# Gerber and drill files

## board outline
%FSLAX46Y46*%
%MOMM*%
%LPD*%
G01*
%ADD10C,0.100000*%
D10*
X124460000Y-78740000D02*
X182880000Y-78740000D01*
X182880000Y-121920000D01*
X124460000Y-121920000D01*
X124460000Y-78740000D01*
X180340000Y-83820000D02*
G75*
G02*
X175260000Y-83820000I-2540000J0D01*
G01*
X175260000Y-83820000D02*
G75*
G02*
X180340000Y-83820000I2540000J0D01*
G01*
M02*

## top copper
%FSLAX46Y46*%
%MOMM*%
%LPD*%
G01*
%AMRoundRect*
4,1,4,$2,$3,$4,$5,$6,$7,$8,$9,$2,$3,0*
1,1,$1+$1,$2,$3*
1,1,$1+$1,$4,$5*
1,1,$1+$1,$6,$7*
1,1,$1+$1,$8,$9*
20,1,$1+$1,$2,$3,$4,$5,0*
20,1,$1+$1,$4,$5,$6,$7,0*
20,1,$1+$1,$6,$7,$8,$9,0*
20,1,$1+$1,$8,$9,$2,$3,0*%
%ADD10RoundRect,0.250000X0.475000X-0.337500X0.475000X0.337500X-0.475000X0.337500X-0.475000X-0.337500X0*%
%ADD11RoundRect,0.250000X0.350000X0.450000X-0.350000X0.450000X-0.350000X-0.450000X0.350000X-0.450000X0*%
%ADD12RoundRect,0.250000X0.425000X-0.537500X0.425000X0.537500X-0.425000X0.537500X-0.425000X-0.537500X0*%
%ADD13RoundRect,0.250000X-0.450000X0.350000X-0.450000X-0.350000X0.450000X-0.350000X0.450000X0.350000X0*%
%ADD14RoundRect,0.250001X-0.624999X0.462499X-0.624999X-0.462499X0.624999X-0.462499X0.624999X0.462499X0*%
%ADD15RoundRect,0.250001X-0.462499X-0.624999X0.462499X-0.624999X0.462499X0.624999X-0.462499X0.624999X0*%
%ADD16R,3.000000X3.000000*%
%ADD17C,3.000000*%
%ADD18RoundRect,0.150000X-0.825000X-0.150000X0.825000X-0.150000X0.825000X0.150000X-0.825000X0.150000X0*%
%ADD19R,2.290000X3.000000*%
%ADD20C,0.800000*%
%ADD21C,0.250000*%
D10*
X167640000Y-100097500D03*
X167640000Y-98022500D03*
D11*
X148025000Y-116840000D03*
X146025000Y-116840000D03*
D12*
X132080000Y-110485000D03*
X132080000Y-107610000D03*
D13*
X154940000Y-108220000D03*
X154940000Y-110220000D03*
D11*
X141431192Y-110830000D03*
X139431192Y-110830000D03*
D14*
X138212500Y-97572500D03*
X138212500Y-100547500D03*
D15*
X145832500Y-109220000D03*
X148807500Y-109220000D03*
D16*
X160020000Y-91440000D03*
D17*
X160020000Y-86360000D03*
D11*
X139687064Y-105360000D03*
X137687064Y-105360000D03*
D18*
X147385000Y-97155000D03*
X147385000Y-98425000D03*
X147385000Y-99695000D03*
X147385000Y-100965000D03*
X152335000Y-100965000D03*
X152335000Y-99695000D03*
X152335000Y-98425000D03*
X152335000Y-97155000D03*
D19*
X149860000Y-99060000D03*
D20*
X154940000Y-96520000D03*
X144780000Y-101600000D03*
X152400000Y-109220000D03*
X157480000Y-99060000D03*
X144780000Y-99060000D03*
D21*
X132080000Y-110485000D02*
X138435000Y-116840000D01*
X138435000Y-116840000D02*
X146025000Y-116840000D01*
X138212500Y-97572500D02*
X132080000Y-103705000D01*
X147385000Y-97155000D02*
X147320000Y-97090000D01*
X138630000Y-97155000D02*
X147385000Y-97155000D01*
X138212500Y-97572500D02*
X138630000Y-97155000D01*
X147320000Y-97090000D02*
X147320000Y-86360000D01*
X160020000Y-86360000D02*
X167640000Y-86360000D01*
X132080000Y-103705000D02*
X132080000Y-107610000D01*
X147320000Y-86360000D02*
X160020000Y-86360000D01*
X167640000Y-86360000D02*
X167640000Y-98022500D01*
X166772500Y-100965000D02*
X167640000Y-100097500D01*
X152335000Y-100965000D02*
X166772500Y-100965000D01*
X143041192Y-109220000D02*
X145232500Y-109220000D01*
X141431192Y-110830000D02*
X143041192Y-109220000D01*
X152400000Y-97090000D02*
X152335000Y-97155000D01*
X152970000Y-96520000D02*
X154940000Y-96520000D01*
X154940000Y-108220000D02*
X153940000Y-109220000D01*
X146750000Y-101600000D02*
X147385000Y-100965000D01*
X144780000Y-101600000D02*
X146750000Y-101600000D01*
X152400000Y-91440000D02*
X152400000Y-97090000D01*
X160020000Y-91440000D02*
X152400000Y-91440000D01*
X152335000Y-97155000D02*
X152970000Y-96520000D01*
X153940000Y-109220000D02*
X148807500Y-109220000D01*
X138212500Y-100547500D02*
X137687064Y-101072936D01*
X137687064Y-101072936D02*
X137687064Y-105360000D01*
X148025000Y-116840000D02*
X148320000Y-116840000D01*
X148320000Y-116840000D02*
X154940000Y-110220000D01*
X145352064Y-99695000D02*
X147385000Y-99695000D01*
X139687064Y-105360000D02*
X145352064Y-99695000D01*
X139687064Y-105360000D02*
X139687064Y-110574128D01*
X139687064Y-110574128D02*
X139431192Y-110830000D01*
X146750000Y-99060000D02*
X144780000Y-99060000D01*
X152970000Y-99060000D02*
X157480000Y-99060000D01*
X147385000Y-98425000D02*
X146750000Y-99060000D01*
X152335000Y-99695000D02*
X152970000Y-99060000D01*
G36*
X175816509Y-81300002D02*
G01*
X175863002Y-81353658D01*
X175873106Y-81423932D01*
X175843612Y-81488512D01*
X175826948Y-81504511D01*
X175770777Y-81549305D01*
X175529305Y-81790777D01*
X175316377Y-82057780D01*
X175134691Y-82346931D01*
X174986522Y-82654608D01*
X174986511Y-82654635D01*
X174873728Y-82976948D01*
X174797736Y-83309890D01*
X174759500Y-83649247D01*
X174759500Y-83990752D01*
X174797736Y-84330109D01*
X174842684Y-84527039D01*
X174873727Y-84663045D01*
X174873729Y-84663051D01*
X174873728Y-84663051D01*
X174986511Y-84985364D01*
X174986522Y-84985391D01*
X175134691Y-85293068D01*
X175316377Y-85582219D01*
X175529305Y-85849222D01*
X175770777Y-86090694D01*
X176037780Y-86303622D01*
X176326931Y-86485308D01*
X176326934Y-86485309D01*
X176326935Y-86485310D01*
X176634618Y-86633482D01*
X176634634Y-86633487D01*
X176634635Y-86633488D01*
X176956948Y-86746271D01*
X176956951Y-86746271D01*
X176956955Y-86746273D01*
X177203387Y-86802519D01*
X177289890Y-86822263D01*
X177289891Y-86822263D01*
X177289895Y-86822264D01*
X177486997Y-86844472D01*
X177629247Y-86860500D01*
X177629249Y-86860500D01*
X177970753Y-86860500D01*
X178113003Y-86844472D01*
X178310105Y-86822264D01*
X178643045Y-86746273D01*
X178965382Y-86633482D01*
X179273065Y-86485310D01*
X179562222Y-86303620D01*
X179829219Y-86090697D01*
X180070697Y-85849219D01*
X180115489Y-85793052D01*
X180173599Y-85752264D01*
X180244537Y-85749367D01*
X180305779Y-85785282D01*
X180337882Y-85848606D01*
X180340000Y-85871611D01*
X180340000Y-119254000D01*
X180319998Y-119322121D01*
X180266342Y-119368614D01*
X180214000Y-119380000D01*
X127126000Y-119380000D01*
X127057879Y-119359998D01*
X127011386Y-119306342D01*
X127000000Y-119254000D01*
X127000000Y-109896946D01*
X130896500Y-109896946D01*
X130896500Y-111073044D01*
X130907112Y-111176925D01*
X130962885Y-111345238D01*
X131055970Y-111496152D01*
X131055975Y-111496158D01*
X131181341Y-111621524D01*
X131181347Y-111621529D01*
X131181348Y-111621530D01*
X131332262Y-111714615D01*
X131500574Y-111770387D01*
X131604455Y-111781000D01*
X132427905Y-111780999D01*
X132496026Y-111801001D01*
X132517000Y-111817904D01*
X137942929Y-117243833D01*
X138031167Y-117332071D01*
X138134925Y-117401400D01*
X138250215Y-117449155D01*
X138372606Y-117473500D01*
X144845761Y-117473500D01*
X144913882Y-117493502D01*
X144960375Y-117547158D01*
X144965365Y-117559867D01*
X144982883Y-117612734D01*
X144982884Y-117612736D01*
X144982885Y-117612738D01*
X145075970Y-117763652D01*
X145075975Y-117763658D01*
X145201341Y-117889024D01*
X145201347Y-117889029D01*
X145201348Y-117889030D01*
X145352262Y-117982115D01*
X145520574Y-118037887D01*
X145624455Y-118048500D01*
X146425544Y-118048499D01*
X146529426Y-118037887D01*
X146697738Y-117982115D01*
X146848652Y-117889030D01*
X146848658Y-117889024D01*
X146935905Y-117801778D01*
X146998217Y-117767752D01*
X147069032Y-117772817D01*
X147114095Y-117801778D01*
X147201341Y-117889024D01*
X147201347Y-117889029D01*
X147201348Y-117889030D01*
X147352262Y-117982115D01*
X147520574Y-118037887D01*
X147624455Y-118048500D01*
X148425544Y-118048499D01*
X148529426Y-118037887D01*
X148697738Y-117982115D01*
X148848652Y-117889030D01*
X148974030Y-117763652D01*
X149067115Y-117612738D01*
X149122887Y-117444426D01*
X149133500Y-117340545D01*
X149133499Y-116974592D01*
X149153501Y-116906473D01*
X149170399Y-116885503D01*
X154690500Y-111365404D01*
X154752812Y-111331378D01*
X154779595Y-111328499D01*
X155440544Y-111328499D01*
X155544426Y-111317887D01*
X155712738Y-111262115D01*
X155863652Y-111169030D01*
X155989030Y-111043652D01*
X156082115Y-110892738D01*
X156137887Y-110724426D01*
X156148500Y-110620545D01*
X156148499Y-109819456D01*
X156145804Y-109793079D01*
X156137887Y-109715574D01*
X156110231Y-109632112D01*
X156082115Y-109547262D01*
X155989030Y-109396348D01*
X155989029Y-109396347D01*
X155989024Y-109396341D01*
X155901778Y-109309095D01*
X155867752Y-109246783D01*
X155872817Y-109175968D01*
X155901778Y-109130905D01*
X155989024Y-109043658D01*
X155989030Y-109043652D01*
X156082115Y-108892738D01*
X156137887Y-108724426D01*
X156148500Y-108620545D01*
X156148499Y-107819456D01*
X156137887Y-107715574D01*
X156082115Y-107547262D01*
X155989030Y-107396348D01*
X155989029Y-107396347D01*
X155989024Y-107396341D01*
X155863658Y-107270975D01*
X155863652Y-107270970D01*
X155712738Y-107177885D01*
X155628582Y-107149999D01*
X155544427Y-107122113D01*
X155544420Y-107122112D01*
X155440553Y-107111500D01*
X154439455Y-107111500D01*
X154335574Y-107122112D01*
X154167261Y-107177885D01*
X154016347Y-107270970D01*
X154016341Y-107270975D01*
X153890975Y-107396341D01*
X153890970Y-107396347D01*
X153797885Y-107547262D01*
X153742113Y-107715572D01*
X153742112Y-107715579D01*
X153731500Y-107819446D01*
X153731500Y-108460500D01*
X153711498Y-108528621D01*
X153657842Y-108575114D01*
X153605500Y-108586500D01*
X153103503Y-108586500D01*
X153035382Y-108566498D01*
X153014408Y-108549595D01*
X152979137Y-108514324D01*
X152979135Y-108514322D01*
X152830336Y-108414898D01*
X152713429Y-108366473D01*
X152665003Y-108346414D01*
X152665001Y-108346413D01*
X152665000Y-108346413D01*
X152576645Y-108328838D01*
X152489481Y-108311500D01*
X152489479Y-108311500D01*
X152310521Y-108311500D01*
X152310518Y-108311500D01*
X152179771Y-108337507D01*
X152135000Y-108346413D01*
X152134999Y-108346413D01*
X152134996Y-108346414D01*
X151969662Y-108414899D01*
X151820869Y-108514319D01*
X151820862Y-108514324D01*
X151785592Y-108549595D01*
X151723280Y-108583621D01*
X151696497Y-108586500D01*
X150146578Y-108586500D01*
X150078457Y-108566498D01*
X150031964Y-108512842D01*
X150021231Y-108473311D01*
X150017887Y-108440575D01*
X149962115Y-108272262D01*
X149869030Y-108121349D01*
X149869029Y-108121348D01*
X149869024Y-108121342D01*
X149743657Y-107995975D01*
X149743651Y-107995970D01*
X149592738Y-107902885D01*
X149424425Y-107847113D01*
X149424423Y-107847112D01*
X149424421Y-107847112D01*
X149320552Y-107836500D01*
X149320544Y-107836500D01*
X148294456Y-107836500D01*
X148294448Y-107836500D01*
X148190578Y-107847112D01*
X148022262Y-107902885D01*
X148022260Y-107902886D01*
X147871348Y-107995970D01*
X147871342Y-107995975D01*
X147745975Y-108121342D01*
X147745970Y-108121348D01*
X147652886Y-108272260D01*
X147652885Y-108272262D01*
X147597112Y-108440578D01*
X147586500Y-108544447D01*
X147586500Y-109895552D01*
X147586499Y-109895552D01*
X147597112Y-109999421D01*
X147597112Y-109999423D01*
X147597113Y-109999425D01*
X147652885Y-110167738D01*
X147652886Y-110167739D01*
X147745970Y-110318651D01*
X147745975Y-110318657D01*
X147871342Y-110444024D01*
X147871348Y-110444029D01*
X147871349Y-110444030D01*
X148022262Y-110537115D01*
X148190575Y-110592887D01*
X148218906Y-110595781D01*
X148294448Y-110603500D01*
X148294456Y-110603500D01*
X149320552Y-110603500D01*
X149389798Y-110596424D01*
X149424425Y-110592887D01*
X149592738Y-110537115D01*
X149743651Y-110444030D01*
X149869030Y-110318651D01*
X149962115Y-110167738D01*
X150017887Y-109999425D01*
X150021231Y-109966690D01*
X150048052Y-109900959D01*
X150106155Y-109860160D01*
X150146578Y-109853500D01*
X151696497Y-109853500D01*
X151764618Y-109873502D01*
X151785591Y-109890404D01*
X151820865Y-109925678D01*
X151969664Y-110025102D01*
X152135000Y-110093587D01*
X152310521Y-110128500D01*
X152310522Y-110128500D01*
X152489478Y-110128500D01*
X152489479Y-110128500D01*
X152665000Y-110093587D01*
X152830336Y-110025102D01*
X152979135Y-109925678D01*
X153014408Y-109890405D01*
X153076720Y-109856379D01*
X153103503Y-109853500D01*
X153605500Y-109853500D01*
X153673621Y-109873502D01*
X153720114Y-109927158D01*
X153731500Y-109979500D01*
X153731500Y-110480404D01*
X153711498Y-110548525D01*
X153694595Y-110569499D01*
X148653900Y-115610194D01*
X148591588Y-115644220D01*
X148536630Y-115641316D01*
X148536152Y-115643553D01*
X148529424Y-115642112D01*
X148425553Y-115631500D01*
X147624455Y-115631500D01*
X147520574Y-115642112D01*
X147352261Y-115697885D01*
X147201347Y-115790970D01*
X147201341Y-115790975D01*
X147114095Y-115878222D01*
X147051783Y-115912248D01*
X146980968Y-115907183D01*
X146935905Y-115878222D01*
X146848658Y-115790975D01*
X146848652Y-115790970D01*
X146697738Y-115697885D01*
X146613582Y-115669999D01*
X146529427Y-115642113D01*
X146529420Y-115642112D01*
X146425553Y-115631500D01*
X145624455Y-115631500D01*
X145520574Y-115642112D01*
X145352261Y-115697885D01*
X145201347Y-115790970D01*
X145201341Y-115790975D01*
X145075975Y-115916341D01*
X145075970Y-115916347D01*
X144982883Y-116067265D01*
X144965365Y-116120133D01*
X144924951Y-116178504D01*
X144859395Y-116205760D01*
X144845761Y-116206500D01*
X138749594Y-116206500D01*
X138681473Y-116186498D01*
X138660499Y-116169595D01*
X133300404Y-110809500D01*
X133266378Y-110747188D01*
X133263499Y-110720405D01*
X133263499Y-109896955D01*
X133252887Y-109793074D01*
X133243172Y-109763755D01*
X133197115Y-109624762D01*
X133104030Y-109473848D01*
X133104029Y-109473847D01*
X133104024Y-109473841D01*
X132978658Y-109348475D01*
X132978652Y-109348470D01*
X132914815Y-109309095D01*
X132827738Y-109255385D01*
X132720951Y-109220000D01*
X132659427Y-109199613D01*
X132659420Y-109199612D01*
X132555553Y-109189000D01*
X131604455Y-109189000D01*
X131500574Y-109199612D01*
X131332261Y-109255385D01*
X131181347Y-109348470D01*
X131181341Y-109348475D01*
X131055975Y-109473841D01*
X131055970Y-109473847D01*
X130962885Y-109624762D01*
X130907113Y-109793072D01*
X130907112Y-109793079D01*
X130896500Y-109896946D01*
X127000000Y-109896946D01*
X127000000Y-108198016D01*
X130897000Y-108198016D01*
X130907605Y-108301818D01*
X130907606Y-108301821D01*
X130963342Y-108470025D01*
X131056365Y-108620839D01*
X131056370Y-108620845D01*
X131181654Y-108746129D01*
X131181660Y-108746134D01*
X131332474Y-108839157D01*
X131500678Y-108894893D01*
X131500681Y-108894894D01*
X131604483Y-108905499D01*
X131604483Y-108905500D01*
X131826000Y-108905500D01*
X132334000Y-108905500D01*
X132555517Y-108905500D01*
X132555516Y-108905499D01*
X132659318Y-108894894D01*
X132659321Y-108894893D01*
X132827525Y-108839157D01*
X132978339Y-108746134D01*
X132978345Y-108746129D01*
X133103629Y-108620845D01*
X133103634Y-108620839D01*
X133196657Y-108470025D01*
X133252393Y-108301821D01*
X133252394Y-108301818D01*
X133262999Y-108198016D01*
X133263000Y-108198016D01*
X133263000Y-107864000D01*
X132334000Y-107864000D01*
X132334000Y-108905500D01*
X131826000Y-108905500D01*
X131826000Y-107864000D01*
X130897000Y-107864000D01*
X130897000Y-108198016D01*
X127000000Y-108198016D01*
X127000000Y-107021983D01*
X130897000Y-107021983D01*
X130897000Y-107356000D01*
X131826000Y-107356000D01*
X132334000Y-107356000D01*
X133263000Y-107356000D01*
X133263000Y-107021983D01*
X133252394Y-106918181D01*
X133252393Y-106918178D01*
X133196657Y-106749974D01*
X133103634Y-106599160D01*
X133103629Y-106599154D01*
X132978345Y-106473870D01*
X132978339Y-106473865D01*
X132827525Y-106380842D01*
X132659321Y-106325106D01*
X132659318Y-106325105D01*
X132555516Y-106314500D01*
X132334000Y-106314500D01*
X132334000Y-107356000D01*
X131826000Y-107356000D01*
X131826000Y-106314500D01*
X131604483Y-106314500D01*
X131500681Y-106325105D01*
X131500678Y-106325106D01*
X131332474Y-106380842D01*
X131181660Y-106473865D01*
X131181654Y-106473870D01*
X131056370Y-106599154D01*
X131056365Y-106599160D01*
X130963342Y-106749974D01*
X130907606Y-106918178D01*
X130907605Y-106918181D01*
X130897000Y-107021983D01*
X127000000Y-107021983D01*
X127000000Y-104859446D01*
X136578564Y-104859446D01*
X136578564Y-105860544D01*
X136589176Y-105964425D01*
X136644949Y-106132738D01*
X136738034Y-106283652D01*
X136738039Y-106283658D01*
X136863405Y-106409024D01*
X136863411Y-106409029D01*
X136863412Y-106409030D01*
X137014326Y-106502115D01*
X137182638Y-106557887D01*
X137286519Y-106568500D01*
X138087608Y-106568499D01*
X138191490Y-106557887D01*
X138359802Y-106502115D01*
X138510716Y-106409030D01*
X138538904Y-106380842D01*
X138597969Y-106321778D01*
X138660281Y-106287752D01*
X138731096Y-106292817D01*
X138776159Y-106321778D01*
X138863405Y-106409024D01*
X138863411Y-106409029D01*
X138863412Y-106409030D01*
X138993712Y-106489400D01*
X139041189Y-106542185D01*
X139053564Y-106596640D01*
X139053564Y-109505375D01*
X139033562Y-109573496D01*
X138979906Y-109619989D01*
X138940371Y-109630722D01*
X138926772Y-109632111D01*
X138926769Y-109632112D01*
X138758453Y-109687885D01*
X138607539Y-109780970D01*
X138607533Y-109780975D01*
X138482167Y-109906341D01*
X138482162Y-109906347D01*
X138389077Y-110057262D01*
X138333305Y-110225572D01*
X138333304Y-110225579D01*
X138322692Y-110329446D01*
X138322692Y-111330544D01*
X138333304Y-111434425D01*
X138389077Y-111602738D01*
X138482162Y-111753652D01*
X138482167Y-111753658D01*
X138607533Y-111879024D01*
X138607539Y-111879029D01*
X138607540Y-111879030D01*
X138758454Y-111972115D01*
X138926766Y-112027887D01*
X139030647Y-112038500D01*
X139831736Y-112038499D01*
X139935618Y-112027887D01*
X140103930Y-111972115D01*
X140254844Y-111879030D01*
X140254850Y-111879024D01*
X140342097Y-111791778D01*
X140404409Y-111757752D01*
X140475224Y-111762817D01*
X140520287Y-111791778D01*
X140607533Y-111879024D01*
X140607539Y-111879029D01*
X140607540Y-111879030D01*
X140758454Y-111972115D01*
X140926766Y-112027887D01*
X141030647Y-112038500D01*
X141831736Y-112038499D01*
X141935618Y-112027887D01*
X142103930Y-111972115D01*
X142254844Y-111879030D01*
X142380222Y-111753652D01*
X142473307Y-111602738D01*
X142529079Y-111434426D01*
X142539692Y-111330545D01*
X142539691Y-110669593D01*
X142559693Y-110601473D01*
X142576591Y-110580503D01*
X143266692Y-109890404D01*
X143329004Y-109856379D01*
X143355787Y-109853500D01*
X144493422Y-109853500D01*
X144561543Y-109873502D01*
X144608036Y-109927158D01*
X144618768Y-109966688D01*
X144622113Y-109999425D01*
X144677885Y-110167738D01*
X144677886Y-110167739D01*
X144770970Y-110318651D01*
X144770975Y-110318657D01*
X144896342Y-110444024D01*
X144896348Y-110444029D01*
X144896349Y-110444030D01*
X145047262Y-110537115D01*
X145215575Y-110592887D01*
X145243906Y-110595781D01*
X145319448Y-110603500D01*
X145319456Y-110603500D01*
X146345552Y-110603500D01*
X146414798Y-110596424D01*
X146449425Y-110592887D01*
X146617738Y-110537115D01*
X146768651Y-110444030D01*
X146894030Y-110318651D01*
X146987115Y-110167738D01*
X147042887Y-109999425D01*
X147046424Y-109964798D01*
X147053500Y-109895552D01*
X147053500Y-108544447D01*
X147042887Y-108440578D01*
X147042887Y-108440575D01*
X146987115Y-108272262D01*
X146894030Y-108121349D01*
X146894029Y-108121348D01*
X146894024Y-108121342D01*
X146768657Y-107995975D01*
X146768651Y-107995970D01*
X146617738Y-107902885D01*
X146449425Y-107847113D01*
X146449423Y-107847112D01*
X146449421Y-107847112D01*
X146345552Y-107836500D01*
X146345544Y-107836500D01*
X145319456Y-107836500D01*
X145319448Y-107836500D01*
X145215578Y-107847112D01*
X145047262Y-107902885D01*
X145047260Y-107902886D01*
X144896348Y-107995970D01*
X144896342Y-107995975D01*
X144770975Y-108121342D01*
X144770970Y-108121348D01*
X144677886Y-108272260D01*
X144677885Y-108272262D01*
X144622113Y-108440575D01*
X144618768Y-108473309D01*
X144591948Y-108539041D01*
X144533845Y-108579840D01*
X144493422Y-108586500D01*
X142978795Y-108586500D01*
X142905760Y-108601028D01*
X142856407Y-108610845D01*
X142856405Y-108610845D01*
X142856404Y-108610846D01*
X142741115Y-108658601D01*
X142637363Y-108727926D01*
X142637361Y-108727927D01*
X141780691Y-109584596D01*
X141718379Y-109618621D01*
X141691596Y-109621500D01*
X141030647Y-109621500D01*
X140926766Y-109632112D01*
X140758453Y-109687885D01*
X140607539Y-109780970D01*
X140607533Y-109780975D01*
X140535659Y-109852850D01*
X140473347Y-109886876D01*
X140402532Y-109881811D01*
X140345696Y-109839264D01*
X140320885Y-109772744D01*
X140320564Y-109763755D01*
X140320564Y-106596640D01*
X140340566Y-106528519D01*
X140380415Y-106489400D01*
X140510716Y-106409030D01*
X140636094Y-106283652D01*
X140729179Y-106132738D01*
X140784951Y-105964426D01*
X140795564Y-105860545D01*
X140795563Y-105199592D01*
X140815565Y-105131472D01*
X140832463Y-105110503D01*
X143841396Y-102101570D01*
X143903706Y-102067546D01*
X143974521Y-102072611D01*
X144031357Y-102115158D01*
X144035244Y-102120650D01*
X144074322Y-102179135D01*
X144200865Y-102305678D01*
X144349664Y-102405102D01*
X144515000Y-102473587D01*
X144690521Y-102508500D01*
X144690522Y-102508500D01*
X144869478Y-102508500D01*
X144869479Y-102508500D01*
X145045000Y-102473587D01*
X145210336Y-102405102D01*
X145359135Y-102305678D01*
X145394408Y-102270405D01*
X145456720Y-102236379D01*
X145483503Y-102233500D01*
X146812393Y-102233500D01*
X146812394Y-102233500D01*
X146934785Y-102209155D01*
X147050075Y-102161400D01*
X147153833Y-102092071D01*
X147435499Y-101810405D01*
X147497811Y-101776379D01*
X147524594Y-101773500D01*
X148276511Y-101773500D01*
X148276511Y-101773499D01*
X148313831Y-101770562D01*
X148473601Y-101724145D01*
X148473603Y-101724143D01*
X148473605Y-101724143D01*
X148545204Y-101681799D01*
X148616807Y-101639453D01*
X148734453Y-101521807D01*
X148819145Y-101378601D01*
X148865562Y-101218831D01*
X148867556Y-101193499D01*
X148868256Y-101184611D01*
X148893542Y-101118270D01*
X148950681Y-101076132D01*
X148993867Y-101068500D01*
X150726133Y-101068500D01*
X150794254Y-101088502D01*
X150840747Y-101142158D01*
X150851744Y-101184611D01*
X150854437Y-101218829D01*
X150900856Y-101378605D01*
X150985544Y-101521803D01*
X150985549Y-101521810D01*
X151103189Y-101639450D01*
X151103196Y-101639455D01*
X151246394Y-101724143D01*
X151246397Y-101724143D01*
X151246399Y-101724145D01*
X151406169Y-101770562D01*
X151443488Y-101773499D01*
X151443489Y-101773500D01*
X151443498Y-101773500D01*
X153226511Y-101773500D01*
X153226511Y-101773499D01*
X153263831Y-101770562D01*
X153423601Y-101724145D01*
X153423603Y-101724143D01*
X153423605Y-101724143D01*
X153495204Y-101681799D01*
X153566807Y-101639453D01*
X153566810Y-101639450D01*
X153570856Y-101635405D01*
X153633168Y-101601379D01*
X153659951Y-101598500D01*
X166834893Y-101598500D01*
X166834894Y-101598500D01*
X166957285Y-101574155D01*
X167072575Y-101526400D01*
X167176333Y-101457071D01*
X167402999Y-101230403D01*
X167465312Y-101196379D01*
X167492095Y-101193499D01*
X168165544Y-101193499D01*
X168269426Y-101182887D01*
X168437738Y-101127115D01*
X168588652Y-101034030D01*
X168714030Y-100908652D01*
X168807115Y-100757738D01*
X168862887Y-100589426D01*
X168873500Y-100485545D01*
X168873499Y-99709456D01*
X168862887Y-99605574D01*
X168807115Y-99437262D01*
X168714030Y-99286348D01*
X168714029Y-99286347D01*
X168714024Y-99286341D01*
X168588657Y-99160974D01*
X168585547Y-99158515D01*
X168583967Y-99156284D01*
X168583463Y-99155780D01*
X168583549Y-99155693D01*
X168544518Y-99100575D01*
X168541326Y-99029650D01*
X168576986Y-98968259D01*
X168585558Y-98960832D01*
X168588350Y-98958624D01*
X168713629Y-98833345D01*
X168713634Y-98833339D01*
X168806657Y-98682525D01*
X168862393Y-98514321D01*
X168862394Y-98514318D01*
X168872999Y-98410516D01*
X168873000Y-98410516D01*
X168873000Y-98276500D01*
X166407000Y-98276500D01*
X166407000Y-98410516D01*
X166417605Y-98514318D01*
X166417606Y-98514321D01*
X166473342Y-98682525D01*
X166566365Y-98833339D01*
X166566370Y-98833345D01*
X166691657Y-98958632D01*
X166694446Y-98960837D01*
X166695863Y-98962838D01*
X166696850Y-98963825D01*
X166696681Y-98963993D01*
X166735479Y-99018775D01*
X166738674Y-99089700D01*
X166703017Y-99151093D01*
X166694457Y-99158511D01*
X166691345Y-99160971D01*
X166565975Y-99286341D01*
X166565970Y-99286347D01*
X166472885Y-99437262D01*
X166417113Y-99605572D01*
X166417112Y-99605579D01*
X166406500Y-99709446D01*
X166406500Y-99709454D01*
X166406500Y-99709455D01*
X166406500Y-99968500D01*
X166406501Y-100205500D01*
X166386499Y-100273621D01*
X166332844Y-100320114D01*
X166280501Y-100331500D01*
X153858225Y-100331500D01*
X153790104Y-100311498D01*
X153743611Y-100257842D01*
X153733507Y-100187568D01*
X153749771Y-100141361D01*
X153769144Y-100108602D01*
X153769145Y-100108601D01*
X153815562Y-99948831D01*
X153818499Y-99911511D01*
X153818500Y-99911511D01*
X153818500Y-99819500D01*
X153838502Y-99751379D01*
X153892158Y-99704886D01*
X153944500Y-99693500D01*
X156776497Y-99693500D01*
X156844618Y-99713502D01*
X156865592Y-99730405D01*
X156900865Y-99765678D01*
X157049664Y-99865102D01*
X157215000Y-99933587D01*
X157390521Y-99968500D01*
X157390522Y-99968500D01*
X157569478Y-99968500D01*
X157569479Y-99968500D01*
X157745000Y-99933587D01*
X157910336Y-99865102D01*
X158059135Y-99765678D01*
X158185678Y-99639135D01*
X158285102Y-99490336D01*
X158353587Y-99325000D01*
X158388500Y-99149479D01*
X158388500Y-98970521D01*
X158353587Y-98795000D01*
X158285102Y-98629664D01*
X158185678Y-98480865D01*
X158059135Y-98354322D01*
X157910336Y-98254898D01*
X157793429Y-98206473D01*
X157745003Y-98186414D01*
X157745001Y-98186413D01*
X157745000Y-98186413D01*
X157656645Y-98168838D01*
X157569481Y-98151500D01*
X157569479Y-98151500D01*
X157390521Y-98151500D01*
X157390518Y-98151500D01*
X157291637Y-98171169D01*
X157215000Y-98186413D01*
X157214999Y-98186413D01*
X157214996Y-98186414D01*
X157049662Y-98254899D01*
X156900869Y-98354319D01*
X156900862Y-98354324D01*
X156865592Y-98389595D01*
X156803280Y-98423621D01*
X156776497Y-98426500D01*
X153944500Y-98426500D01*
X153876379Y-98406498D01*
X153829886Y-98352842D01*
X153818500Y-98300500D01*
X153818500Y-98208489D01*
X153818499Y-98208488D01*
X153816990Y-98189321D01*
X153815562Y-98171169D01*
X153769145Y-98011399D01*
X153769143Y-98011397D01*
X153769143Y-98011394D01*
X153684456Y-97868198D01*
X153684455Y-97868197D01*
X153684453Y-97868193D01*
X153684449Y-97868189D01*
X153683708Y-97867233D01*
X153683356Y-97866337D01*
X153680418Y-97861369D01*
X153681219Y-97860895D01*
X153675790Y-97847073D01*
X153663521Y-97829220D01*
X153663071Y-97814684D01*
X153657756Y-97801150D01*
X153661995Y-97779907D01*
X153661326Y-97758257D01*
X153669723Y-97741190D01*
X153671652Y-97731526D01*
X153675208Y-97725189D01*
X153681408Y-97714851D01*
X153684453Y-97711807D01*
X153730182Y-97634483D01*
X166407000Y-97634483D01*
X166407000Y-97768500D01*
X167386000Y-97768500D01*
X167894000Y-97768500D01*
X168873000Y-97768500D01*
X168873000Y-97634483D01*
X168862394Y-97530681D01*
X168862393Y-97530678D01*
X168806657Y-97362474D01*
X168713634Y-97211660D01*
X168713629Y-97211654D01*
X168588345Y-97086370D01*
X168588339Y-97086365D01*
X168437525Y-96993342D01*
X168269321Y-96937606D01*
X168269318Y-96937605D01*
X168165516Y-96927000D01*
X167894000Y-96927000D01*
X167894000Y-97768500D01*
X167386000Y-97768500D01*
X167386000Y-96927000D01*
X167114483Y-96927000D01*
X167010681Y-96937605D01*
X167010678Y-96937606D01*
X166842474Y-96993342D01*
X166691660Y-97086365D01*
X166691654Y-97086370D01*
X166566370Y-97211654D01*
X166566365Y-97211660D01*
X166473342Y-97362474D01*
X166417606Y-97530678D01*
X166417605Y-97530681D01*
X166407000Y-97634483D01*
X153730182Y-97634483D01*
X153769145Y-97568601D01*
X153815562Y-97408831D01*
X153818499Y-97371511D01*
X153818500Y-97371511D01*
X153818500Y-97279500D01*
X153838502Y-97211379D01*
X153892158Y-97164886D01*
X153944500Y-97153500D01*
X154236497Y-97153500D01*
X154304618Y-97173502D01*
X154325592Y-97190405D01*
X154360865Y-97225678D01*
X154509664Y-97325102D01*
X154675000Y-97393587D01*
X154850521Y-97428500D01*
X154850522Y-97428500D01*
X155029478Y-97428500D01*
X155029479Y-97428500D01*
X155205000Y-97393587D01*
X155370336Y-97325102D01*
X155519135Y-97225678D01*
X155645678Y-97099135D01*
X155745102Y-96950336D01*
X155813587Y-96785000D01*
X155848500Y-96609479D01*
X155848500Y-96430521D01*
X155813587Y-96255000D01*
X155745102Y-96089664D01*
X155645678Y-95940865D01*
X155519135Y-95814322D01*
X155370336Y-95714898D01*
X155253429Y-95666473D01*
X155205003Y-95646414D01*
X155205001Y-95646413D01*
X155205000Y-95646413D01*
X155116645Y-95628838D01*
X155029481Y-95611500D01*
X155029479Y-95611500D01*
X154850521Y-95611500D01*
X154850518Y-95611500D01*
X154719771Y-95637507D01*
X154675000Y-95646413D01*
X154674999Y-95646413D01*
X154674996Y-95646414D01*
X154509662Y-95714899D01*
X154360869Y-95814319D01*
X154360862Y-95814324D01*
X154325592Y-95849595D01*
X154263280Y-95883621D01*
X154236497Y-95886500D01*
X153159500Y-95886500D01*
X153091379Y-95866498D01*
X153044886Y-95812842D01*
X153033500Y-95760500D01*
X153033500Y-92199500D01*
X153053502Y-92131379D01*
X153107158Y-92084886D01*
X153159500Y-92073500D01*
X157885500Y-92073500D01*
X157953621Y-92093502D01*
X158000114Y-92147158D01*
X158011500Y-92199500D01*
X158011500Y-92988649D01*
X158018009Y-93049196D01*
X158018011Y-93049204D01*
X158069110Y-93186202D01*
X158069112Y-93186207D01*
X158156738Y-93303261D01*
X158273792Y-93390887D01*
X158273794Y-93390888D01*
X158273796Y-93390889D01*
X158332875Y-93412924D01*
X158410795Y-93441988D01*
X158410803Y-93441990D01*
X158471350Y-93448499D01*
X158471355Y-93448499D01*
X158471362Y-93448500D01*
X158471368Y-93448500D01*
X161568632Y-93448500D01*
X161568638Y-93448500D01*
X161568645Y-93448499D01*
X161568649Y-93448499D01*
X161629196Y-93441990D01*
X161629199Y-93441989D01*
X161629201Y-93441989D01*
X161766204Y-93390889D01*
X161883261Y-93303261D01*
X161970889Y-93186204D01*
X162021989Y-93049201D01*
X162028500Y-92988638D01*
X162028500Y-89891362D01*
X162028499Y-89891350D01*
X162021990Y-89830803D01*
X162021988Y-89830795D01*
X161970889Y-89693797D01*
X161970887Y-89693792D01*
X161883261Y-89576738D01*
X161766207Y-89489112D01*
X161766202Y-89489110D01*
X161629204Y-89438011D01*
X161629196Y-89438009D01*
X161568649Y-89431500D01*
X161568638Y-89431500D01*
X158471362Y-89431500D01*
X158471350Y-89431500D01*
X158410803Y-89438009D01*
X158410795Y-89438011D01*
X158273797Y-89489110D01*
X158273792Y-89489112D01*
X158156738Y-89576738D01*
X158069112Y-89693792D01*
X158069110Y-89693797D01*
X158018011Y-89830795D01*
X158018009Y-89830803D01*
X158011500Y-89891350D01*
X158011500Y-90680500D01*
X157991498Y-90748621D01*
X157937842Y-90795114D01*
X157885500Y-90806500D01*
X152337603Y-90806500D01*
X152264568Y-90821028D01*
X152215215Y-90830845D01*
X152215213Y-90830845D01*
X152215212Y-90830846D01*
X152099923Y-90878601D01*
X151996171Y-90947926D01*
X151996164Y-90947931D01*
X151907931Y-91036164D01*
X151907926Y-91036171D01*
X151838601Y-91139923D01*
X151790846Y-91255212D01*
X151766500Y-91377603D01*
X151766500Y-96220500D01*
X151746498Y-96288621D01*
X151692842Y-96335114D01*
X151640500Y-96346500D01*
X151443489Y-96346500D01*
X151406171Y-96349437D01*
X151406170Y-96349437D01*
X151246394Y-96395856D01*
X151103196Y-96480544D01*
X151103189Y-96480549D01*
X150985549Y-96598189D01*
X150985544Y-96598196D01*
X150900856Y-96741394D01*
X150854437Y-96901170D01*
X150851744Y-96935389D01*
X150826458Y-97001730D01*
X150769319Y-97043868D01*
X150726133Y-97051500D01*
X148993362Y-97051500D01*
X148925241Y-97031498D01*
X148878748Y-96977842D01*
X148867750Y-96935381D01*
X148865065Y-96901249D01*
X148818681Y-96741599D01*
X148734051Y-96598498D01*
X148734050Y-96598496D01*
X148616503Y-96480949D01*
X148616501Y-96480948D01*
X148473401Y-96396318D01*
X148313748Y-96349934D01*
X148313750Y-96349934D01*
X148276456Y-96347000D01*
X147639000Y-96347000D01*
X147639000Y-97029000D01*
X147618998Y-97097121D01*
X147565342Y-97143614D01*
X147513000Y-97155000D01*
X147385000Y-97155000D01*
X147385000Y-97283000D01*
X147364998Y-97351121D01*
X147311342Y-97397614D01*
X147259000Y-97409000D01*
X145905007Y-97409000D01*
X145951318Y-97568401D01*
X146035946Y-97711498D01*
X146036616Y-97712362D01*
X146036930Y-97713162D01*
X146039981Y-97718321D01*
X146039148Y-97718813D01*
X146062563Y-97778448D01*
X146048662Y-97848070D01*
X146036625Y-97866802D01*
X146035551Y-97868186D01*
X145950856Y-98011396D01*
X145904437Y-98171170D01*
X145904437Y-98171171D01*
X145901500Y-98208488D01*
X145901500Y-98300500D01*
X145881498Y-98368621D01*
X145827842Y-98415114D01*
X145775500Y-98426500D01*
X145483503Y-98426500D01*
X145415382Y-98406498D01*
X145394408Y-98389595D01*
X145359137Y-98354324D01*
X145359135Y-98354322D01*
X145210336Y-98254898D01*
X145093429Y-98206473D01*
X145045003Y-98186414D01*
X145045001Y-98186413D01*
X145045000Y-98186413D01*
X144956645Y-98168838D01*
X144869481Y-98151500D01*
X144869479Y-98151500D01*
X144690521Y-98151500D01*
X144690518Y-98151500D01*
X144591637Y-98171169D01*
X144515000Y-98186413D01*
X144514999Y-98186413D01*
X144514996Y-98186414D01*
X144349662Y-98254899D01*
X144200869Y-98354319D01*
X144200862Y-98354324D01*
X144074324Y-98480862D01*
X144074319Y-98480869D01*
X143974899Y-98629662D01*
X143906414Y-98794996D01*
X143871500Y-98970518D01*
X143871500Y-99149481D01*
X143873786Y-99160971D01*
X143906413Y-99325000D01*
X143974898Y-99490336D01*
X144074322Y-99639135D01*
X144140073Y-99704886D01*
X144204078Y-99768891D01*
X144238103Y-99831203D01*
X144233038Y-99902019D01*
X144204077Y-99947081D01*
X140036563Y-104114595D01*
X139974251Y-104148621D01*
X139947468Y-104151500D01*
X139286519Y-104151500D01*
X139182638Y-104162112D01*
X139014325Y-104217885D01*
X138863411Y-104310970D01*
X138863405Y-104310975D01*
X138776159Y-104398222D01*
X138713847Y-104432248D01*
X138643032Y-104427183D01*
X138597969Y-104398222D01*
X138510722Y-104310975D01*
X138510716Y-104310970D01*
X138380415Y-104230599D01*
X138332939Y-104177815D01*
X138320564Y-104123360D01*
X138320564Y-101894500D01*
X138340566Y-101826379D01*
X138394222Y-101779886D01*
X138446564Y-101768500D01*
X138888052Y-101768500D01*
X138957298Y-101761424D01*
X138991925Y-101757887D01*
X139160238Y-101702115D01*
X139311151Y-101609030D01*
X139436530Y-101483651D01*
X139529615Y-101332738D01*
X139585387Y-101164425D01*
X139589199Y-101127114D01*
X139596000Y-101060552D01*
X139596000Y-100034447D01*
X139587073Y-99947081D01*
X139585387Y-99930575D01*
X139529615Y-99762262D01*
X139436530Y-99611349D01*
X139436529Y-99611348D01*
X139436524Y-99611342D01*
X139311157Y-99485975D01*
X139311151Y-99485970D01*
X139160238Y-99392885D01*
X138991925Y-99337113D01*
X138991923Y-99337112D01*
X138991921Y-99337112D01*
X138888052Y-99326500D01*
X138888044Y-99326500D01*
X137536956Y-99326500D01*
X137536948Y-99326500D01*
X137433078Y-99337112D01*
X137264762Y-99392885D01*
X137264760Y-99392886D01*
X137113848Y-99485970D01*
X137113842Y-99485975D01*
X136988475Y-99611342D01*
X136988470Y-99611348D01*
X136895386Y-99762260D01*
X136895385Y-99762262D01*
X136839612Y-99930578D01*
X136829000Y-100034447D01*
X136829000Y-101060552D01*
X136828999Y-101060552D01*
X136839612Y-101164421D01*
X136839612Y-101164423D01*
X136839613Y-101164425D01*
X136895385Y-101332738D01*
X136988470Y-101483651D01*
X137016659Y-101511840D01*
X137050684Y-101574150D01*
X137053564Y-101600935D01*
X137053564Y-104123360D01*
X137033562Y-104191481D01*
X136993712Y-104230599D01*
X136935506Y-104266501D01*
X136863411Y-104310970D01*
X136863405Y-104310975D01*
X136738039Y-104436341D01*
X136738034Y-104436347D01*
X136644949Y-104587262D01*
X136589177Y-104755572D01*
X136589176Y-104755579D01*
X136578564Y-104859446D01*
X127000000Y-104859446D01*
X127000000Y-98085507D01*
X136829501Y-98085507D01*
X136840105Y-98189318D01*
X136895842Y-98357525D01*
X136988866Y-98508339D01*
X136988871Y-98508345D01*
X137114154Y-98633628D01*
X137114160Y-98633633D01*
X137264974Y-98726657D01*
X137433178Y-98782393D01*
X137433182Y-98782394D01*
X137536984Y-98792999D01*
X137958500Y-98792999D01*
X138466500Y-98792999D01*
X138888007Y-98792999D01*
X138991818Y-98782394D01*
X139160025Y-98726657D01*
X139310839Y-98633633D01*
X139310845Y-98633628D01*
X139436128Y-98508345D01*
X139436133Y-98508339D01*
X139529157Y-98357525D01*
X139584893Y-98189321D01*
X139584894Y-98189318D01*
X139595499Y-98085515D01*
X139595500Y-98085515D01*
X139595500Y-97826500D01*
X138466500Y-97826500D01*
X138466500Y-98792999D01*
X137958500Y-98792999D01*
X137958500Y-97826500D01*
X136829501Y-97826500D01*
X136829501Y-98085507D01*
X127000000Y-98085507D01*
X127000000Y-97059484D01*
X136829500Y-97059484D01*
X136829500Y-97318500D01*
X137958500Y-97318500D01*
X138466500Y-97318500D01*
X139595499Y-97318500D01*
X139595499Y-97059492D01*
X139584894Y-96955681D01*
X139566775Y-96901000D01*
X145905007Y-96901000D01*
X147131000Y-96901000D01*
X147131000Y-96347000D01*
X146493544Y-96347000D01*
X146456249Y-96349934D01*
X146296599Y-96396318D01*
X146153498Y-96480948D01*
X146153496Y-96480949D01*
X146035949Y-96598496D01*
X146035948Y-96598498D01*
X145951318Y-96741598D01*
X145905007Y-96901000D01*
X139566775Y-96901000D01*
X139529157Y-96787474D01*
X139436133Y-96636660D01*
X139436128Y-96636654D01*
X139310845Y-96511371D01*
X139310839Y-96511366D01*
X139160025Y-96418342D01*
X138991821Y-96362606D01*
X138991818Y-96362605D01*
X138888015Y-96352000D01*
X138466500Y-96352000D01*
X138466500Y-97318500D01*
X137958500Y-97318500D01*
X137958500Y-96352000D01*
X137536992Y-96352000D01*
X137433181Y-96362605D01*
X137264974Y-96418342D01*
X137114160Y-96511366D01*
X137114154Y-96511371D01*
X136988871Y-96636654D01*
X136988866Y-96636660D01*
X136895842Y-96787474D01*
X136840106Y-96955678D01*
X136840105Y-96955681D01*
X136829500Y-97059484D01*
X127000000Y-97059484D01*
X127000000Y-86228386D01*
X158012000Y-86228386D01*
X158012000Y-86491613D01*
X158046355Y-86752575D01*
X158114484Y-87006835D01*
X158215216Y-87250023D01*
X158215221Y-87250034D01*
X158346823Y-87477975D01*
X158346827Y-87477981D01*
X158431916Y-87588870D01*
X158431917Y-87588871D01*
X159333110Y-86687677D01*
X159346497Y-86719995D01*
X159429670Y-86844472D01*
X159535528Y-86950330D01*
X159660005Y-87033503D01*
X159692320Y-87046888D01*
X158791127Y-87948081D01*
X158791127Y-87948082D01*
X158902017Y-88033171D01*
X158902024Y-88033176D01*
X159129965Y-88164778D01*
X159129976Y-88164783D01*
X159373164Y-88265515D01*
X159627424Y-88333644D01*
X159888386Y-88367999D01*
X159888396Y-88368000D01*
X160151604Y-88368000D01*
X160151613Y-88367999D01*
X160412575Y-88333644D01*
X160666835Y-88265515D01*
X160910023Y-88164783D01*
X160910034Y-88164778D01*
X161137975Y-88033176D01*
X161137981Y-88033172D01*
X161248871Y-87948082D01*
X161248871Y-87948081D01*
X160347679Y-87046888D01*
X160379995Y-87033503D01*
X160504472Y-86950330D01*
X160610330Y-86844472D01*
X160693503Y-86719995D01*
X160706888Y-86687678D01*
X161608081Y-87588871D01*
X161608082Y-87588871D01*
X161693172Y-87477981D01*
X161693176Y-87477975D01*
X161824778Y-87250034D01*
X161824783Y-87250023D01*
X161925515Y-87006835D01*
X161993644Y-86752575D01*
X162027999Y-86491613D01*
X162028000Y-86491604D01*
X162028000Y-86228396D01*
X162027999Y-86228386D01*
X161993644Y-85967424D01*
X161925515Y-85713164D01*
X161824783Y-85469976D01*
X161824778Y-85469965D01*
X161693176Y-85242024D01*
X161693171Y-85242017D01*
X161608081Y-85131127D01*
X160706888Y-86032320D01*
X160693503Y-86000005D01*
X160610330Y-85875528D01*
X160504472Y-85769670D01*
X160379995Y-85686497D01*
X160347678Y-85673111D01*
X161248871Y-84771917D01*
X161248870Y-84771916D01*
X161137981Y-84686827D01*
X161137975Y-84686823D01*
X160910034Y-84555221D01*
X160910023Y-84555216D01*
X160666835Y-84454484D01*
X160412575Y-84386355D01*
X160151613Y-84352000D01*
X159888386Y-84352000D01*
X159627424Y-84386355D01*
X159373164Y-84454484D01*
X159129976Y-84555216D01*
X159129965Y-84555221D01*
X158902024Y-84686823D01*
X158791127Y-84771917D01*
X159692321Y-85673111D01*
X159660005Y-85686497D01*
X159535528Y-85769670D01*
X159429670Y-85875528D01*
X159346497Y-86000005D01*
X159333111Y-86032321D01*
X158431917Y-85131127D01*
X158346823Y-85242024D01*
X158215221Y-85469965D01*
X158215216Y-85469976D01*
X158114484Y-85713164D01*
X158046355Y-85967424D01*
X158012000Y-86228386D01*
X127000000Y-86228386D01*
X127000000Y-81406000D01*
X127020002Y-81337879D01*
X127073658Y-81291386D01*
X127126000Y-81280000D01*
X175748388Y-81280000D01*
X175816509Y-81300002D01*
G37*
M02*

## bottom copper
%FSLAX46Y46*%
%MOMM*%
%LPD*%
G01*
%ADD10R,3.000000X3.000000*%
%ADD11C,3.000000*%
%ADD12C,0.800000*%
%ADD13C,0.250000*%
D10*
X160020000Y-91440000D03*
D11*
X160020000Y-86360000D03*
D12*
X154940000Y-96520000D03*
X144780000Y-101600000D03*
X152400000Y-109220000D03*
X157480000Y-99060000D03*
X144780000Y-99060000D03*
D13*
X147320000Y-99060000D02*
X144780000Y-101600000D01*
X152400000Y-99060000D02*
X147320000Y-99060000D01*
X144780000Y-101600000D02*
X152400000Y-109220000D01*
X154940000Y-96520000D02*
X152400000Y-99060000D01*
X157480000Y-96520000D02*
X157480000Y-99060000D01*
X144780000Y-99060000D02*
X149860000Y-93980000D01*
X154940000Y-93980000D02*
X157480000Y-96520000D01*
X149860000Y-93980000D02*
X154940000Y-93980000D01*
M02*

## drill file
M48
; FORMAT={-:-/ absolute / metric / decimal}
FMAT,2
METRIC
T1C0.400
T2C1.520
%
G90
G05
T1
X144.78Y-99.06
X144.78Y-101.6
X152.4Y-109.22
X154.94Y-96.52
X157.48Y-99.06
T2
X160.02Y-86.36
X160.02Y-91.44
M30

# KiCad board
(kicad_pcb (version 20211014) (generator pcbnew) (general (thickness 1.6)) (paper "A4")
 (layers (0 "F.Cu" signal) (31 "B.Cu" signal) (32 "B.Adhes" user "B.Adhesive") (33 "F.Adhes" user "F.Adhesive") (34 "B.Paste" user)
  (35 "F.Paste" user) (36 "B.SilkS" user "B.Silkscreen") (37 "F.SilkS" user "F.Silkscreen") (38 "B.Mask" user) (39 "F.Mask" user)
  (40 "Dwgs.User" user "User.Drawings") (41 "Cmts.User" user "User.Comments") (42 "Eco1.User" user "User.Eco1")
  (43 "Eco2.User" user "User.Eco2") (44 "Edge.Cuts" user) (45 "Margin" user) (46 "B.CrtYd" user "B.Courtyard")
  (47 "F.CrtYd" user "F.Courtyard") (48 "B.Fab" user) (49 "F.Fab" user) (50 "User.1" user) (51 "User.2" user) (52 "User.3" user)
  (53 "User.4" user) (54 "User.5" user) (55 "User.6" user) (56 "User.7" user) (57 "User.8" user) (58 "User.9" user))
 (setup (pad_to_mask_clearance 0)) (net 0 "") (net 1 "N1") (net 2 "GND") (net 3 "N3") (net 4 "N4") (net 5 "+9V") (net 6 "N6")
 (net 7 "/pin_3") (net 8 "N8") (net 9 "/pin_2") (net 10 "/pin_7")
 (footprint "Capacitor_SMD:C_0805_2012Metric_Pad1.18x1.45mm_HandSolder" (layer "F.Cu") (at 167.64 99.06 90)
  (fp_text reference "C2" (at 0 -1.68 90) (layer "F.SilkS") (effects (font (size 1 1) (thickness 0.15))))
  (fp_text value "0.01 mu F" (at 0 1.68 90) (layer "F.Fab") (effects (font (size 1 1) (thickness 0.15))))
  (pad "1" smd roundrect (at -1.0375 0 90) (size 1.175 1.45) (layers "F.Cu" "F.Paste" "F.Mask") (roundrect_rratio 0.2127659574) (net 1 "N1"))
  (pad "2" smd roundrect (at 1.0375 0 90) (size 1.175 1.45) (layers "F.Cu" "F.Paste" "F.Mask") (roundrect_rratio 0.2127659574) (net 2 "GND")))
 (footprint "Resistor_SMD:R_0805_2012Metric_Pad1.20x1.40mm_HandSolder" (layer "F.Cu") (at 147.025 116.84 180)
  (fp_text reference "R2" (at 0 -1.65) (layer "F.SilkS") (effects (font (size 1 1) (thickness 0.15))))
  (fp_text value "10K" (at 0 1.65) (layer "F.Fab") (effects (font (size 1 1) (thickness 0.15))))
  (pad "1" smd roundrect (at -1 0 180) (size 1.2 1.4) (layers "F.Cu" "F.Paste" "F.Mask") (roundrect_rratio 0.2083333333) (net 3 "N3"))
  (pad "2" smd roundrect (at 1 0 180) (size 1.2 1.4) (layers "F.Cu" "F.Paste" "F.Mask") (roundrect_rratio 0.2083333333) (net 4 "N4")))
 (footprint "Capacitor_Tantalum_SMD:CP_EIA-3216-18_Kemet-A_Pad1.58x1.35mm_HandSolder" (layer "F.Cu") (at 132.08 109.0475 90)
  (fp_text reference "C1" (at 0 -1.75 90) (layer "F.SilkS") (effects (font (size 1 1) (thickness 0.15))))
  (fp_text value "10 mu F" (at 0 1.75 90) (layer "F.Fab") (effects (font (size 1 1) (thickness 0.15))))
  (pad "1" smd roundrect (at -1.4375 0 90) (size 1.575 1.35) (layers "F.Cu" "F.Paste" "F.Mask") (roundrect_rratio 0.1851851852) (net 4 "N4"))
  (pad "2" smd roundrect (at 1.4375 0 90) (size 1.575 1.35) (layers "F.Cu" "F.Paste" "F.Mask") (roundrect_rratio 0.1851851852) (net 2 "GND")))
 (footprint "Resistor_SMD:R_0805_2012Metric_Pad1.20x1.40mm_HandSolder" (layer "F.Cu") (at 154.94 109.22 -90)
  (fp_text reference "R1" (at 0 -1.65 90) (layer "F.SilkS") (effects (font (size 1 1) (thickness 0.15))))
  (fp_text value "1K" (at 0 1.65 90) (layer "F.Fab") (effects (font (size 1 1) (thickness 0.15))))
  (pad "1" smd roundrect (at -1 0 270) (size 1.2 1.4) (layers "F.Cu" "F.Paste" "F.Mask") (roundrect_rratio 0.2083333333) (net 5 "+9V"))
  (pad "2" smd roundrect (at 1 0 270) (size 1.2 1.4) (layers "F.Cu" "F.Paste" "F.Mask") (roundrect_rratio 0.2083333333) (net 3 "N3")))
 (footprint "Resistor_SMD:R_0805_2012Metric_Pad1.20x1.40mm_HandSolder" (layer "F.Cu") (at 140.431192 110.83 180)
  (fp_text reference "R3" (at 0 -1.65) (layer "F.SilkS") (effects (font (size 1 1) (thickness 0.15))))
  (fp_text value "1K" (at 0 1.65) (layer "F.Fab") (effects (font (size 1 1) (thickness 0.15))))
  (pad "1" smd roundrect (at -1 0 180) (size 1.2 1.4) (layers "F.Cu" "F.Paste" "F.Mask") (roundrect_rratio 0.2083333333) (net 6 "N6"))
  (pad "2" smd roundrect (at 1 0 180) (size 1.2 1.4) (layers "F.Cu" "F.Paste" "F.Mask") (roundrect_rratio 0.2083333333) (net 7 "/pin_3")))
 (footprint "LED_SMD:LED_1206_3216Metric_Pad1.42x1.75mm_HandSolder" (layer "F.Cu") (at 138.2125 99.06 -90)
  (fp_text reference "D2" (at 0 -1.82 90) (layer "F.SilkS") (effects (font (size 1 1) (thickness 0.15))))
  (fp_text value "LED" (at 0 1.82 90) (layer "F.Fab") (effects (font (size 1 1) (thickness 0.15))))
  (pad "1" smd roundrect (at -1.4875 0 270) (size 1.425 1.75) (layers "F.Cu" "F.Paste" "F.Mask") (roundrect_rratio 0.1754392982)
   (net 2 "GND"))
  (pad "2" smd roundrect (at 1.4875 0 270) (size 1.425 1.75) (layers "F.Cu" "F.Paste" "F.Mask") (roundrect_rratio 0.1754392982) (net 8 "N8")))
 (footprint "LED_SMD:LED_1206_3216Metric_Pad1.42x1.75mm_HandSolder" (layer "F.Cu") (at 147.32 109.22)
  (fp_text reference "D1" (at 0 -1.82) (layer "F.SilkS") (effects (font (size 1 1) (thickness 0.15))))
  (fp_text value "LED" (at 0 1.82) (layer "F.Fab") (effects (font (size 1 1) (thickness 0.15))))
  (pad "1" smd roundrect (at -1.4875 0) (size 1.425 1.75) (layers "F.Cu" "F.Paste" "F.Mask") (roundrect_rratio 0.1754392982) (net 6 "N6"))
  (pad "2" smd roundrect (at 1.4875 0) (size 1.425 1.75) (layers "F.Cu" "F.Paste" "F.Mask") (roundrect_rratio 0.1754392982) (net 5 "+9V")))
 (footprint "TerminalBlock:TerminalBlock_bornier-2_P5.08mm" (layer "F.Cu") (at 160.02 91.44 90)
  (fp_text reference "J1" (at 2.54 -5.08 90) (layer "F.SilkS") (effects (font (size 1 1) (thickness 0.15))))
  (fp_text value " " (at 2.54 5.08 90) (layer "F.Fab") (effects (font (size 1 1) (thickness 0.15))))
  (pad "1" thru_hole rect (at 0 0 90) (size 3 3) (drill 1.52) (layers *.Cu *.Mask) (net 5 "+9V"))
  (pad "2" thru_hole circle (at 5.08 0 90) (size 3 3) (drill 1.52) (layers *.Cu *.Mask) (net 2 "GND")))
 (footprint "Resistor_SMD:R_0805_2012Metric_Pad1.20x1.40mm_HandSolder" (layer "F.Cu") (at 138.687064 105.36 180)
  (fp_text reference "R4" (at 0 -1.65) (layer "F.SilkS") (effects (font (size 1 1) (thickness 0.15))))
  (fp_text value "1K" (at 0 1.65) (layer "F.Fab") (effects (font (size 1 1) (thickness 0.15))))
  (pad "1" smd roundrect (at -1 0 180) (size 1.2 1.4) (layers "F.Cu" "F.Paste" "F.Mask") (roundrect_rratio 0.2083333333) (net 7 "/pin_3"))
  (pad "2" smd roundrect (at 1 0 180) (size 1.2 1.4) (layers "F.Cu" "F.Paste" "F.Mask") (roundrect_rratio 0.2083333333) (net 8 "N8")))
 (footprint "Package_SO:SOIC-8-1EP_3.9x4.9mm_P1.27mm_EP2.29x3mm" (layer "F.Cu") (at 149.86 99.06)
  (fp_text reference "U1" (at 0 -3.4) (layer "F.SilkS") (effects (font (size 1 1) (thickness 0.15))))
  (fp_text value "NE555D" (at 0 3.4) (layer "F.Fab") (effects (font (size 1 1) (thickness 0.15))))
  (pad "" smd roundrect (at -0.57 0.75) (size 0.92 1.21) (layers "F.Paste") (roundrect_rratio 0.25))
  (pad "" smd roundrect (at 0.57 -0.75) (size 0.92 1.21) (layers "F.Paste") (roundrect_rratio 0.25))
  (pad "" smd roundrect (at 0.57 0.75) (size 0.92 1.21) (layers "F.Paste") (roundrect_rratio 0.25))
  (pad "" smd roundrect (at -0.57 -0.75) (size 0.92 1.21) (layers "F.Paste") (roundrect_rratio 0.25))
  (pad "1" smd roundrect (at -2.475 -1.905) (size 1.95 0.6) (layers "F.Cu" "F.Paste" "F.Mask") (roundrect_rratio 0.25) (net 2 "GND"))
  (pad "2" smd roundrect (at -2.475 -0.635) (size 1.95 0.6) (layers "F.Cu" "F.Paste" "F.Mask") (roundrect_rratio 0.25) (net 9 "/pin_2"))
  (pad "3" smd roundrect (at -2.475 0.635) (size 1.95 0.6) (layers "F.Cu" "F.Paste" "F.Mask") (roundrect_rratio 0.25) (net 7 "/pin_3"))
  (pad "4" smd roundrect (at -2.475 1.905) (size 1.95 0.6) (layers "F.Cu" "F.Paste" "F.Mask") (roundrect_rratio 0.25) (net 5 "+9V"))
  (pad "5" smd roundrect (at 2.475 1.905) (size 1.95 0.6) (layers "F.Cu" "F.Paste" "F.Mask") (roundrect_rratio 0.25) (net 1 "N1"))
  (pad "6" smd roundrect (at 2.475 0.635) (size 1.95 0.6) (layers "F.Cu" "F.Paste" "F.Mask") (roundrect_rratio 0.25) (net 9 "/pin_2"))
  (pad "7" smd roundrect (at 2.475 -0.635) (size 1.95 0.6) (layers "F.Cu" "F.Paste" "F.Mask") (roundrect_rratio 0.25) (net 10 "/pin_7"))
  (pad "8" smd roundrect (at 2.475 -1.905) (size 1.95 0.6) (layers "F.Cu" "F.Paste" "F.Mask") (roundrect_rratio 0.25) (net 5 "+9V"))
  (pad "9" smd rect (at 0 0) (size 2.29 3) (layers "F.Cu" "F.Mask")))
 (gr_rect (start 124.46 78.74) (end 182.88 121.92) (layer "Edge.Cuts") (width 0.1) (fill none))
 (gr_circle (center 177.8 83.82) (end 180.34 83.82) (layer "Edge.Cuts") (width 0.1) (fill none))
 (segment (start 132.08 110.485) (end 138.435 116.84) (width 0.25) (layer "F.Cu") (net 4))
 (segment (start 138.435 116.84) (end 146.025 116.84) (width 0.25) (layer "F.Cu") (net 4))
 (segment (start 138.2125 97.5725) (end 132.08 103.705) (width 0.25) (layer "F.Cu") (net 2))
 (segment (start 147.385 97.155) (end 147.32 97.09) (width 0.25) (layer "F.Cu") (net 2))
 (segment (start 138.63 97.155) (end 147.385 97.155) (width 0.25) (layer "F.Cu") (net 2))
 (segment (start 138.2125 97.5725) (end 138.63 97.155) (width 0.25) (layer "F.Cu") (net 2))
 (segment (start 147.32 97.09) (end 147.32 86.36) (width 0.25) (layer "F.Cu") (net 2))
 (segment (start 160.02 86.36) (end 167.64 86.36) (width 0.25) (layer "F.Cu") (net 2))
 (segment (start 132.08 103.705) (end 132.08 107.61) (width 0.25) (layer "F.Cu") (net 2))
 (segment (start 147.32 86.36) (end 160.02 86.36) (width 0.25) (layer "F.Cu") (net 2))
 (segment (start 167.64 86.36) (end 167.64 98.0225) (width 0.25) (layer "F.Cu") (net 2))
 (segment (start 166.7725 100.965) (end 167.64 100.0975) (width 0.25) (layer "F.Cu") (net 1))
 (segment (start 152.335 100.965) (end 166.7725 100.965) (width 0.25) (layer "F.Cu") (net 1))
 (segment (start 143.041192 109.22) (end 145.2325 109.22) (width 0.25) (layer "F.Cu") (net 6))
 (segment (start 141.431192 110.83) (end 143.041192 109.22) (width 0.25) (layer "F.Cu") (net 6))
 (segment (start 152.4 97.09) (end 152.335 97.155) (width 0.25) (layer "F.Cu") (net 5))
 (segment (start 152.97 96.52) (end 154.94 96.52) (width 0.25) (layer "F.Cu") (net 5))
 (segment (start 154.94 108.22) (end 153.94 109.22) (width 0.25) (layer "F.Cu") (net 5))
 (segment (start 146.75 101.6) (end 147.385 100.965) (width 0.25) (layer "F.Cu") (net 5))
 (segment (start 144.78 101.6) (end 146.75 101.6) (width 0.25) (layer "F.Cu") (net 5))
 (segment (start 152.4 91.44) (end 152.4 97.09) (width 0.25) (layer "F.Cu") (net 5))
 (segment (start 160.02 91.44) (end 152.4 91.44) (width 0.25) (layer "F.Cu") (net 5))
 (segment (start 152.335 97.155) (end 152.97 96.52) (width 0.25) (layer "F.Cu") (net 5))
 (segment (start 153.94 109.22) (end 148.8075 109.22) (width 0.25) (layer "F.Cu") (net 5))
 (via (at 154.94 96.52) (size 0.8) (drill 0.4) (layers "F.Cu" "B.Cu") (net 5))
 (via (at 144.78 101.6) (size 0.8) (drill 0.4) (layers "F.Cu" "B.Cu") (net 5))
 (via (at 152.4 109.22) (size 0.8) (drill 0.4) (layers "F.Cu" "B.Cu") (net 5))
 (segment (start 147.32 99.06) (end 144.78 101.6) (width 0.25) (layer "B.Cu") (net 5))
 (segment (start 152.4 99.06) (end 147.32 99.06) (width 0.25) (layer "B.Cu") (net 5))
 (segment (start 144.78 101.6) (end 152.4 109.22) (width 0.25) (layer "B.Cu") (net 5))
 (segment (start 154.94 96.52) (end 152.4 99.06) (width 0.25) (layer "B.Cu") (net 5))
 (segment (start 138.2125 100.5475) (end 137.687064 101.072936) (width 0.25) (layer "F.Cu") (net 8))
 (segment (start 137.687064 101.072936) (end 137.687064 105.36) (width 0.25) (layer "F.Cu") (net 8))
 (segment (start 148.025 116.84) (end 148.32 116.84) (width 0.25) (layer "F.Cu") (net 3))
 (segment (start 148.32 116.84) (end 154.94 110.22) (width 0.25) (layer "F.Cu") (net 3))
 (segment (start 145.352064 99.695) (end 147.385 99.695) (width 0.25) (layer "F.Cu") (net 7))
 (segment (start 139.687064 105.36) (end 145.352064 99.695) (width 0.25) (layer "F.Cu") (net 7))
 (segment (start 139.687064 105.36) (end 139.687064 110.574128) (width 0.25) (layer "F.Cu") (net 7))
 (segment (start 139.687064 110.574128) (end 139.431192 110.83) (width 0.25) (layer "F.Cu") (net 7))
 (segment (start 146.75 99.06) (end 144.78 99.06) (width 0.25) (layer "F.Cu") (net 9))
 (segment (start 152.97 99.06) (end 157.48 99.06) (width 0.25) (layer "F.Cu") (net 9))
 (segment (start 147.385 98.425) (end 146.75 99.06) (width 0.25) (layer "F.Cu") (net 9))
 (segment (start 152.335 99.695) (end 152.97 99.06) (width 0.25) (layer "F.Cu") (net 9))
 (via (at 157.48 99.06) (size 0.8) (drill 0.4) (layers "F.Cu" "B.Cu") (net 9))
 (via (at 144.78 99.06) (size 0.8) (drill 0.4) (layers "F.Cu" "B.Cu") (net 9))
 (segment (start 157.48 96.52) (end 157.48 99.06) (width 0.25) (layer "B.Cu") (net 9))
 (segment (start 144.78 99.06) (end 149.86 93.98) (width 0.25) (layer "B.Cu") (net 9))
 (segment (start 154.94 93.98) (end 157.48 96.52) (width 0.25) (layer "B.Cu") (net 9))
 (segment (start 149.86 93.98) (end 154.94 93.98) (width 0.25) (layer "B.Cu") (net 9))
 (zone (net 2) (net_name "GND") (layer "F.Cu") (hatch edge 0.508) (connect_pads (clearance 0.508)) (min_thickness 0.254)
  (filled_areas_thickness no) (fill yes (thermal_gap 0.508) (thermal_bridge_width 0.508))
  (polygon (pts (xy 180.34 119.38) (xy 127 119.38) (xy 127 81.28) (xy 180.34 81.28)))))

